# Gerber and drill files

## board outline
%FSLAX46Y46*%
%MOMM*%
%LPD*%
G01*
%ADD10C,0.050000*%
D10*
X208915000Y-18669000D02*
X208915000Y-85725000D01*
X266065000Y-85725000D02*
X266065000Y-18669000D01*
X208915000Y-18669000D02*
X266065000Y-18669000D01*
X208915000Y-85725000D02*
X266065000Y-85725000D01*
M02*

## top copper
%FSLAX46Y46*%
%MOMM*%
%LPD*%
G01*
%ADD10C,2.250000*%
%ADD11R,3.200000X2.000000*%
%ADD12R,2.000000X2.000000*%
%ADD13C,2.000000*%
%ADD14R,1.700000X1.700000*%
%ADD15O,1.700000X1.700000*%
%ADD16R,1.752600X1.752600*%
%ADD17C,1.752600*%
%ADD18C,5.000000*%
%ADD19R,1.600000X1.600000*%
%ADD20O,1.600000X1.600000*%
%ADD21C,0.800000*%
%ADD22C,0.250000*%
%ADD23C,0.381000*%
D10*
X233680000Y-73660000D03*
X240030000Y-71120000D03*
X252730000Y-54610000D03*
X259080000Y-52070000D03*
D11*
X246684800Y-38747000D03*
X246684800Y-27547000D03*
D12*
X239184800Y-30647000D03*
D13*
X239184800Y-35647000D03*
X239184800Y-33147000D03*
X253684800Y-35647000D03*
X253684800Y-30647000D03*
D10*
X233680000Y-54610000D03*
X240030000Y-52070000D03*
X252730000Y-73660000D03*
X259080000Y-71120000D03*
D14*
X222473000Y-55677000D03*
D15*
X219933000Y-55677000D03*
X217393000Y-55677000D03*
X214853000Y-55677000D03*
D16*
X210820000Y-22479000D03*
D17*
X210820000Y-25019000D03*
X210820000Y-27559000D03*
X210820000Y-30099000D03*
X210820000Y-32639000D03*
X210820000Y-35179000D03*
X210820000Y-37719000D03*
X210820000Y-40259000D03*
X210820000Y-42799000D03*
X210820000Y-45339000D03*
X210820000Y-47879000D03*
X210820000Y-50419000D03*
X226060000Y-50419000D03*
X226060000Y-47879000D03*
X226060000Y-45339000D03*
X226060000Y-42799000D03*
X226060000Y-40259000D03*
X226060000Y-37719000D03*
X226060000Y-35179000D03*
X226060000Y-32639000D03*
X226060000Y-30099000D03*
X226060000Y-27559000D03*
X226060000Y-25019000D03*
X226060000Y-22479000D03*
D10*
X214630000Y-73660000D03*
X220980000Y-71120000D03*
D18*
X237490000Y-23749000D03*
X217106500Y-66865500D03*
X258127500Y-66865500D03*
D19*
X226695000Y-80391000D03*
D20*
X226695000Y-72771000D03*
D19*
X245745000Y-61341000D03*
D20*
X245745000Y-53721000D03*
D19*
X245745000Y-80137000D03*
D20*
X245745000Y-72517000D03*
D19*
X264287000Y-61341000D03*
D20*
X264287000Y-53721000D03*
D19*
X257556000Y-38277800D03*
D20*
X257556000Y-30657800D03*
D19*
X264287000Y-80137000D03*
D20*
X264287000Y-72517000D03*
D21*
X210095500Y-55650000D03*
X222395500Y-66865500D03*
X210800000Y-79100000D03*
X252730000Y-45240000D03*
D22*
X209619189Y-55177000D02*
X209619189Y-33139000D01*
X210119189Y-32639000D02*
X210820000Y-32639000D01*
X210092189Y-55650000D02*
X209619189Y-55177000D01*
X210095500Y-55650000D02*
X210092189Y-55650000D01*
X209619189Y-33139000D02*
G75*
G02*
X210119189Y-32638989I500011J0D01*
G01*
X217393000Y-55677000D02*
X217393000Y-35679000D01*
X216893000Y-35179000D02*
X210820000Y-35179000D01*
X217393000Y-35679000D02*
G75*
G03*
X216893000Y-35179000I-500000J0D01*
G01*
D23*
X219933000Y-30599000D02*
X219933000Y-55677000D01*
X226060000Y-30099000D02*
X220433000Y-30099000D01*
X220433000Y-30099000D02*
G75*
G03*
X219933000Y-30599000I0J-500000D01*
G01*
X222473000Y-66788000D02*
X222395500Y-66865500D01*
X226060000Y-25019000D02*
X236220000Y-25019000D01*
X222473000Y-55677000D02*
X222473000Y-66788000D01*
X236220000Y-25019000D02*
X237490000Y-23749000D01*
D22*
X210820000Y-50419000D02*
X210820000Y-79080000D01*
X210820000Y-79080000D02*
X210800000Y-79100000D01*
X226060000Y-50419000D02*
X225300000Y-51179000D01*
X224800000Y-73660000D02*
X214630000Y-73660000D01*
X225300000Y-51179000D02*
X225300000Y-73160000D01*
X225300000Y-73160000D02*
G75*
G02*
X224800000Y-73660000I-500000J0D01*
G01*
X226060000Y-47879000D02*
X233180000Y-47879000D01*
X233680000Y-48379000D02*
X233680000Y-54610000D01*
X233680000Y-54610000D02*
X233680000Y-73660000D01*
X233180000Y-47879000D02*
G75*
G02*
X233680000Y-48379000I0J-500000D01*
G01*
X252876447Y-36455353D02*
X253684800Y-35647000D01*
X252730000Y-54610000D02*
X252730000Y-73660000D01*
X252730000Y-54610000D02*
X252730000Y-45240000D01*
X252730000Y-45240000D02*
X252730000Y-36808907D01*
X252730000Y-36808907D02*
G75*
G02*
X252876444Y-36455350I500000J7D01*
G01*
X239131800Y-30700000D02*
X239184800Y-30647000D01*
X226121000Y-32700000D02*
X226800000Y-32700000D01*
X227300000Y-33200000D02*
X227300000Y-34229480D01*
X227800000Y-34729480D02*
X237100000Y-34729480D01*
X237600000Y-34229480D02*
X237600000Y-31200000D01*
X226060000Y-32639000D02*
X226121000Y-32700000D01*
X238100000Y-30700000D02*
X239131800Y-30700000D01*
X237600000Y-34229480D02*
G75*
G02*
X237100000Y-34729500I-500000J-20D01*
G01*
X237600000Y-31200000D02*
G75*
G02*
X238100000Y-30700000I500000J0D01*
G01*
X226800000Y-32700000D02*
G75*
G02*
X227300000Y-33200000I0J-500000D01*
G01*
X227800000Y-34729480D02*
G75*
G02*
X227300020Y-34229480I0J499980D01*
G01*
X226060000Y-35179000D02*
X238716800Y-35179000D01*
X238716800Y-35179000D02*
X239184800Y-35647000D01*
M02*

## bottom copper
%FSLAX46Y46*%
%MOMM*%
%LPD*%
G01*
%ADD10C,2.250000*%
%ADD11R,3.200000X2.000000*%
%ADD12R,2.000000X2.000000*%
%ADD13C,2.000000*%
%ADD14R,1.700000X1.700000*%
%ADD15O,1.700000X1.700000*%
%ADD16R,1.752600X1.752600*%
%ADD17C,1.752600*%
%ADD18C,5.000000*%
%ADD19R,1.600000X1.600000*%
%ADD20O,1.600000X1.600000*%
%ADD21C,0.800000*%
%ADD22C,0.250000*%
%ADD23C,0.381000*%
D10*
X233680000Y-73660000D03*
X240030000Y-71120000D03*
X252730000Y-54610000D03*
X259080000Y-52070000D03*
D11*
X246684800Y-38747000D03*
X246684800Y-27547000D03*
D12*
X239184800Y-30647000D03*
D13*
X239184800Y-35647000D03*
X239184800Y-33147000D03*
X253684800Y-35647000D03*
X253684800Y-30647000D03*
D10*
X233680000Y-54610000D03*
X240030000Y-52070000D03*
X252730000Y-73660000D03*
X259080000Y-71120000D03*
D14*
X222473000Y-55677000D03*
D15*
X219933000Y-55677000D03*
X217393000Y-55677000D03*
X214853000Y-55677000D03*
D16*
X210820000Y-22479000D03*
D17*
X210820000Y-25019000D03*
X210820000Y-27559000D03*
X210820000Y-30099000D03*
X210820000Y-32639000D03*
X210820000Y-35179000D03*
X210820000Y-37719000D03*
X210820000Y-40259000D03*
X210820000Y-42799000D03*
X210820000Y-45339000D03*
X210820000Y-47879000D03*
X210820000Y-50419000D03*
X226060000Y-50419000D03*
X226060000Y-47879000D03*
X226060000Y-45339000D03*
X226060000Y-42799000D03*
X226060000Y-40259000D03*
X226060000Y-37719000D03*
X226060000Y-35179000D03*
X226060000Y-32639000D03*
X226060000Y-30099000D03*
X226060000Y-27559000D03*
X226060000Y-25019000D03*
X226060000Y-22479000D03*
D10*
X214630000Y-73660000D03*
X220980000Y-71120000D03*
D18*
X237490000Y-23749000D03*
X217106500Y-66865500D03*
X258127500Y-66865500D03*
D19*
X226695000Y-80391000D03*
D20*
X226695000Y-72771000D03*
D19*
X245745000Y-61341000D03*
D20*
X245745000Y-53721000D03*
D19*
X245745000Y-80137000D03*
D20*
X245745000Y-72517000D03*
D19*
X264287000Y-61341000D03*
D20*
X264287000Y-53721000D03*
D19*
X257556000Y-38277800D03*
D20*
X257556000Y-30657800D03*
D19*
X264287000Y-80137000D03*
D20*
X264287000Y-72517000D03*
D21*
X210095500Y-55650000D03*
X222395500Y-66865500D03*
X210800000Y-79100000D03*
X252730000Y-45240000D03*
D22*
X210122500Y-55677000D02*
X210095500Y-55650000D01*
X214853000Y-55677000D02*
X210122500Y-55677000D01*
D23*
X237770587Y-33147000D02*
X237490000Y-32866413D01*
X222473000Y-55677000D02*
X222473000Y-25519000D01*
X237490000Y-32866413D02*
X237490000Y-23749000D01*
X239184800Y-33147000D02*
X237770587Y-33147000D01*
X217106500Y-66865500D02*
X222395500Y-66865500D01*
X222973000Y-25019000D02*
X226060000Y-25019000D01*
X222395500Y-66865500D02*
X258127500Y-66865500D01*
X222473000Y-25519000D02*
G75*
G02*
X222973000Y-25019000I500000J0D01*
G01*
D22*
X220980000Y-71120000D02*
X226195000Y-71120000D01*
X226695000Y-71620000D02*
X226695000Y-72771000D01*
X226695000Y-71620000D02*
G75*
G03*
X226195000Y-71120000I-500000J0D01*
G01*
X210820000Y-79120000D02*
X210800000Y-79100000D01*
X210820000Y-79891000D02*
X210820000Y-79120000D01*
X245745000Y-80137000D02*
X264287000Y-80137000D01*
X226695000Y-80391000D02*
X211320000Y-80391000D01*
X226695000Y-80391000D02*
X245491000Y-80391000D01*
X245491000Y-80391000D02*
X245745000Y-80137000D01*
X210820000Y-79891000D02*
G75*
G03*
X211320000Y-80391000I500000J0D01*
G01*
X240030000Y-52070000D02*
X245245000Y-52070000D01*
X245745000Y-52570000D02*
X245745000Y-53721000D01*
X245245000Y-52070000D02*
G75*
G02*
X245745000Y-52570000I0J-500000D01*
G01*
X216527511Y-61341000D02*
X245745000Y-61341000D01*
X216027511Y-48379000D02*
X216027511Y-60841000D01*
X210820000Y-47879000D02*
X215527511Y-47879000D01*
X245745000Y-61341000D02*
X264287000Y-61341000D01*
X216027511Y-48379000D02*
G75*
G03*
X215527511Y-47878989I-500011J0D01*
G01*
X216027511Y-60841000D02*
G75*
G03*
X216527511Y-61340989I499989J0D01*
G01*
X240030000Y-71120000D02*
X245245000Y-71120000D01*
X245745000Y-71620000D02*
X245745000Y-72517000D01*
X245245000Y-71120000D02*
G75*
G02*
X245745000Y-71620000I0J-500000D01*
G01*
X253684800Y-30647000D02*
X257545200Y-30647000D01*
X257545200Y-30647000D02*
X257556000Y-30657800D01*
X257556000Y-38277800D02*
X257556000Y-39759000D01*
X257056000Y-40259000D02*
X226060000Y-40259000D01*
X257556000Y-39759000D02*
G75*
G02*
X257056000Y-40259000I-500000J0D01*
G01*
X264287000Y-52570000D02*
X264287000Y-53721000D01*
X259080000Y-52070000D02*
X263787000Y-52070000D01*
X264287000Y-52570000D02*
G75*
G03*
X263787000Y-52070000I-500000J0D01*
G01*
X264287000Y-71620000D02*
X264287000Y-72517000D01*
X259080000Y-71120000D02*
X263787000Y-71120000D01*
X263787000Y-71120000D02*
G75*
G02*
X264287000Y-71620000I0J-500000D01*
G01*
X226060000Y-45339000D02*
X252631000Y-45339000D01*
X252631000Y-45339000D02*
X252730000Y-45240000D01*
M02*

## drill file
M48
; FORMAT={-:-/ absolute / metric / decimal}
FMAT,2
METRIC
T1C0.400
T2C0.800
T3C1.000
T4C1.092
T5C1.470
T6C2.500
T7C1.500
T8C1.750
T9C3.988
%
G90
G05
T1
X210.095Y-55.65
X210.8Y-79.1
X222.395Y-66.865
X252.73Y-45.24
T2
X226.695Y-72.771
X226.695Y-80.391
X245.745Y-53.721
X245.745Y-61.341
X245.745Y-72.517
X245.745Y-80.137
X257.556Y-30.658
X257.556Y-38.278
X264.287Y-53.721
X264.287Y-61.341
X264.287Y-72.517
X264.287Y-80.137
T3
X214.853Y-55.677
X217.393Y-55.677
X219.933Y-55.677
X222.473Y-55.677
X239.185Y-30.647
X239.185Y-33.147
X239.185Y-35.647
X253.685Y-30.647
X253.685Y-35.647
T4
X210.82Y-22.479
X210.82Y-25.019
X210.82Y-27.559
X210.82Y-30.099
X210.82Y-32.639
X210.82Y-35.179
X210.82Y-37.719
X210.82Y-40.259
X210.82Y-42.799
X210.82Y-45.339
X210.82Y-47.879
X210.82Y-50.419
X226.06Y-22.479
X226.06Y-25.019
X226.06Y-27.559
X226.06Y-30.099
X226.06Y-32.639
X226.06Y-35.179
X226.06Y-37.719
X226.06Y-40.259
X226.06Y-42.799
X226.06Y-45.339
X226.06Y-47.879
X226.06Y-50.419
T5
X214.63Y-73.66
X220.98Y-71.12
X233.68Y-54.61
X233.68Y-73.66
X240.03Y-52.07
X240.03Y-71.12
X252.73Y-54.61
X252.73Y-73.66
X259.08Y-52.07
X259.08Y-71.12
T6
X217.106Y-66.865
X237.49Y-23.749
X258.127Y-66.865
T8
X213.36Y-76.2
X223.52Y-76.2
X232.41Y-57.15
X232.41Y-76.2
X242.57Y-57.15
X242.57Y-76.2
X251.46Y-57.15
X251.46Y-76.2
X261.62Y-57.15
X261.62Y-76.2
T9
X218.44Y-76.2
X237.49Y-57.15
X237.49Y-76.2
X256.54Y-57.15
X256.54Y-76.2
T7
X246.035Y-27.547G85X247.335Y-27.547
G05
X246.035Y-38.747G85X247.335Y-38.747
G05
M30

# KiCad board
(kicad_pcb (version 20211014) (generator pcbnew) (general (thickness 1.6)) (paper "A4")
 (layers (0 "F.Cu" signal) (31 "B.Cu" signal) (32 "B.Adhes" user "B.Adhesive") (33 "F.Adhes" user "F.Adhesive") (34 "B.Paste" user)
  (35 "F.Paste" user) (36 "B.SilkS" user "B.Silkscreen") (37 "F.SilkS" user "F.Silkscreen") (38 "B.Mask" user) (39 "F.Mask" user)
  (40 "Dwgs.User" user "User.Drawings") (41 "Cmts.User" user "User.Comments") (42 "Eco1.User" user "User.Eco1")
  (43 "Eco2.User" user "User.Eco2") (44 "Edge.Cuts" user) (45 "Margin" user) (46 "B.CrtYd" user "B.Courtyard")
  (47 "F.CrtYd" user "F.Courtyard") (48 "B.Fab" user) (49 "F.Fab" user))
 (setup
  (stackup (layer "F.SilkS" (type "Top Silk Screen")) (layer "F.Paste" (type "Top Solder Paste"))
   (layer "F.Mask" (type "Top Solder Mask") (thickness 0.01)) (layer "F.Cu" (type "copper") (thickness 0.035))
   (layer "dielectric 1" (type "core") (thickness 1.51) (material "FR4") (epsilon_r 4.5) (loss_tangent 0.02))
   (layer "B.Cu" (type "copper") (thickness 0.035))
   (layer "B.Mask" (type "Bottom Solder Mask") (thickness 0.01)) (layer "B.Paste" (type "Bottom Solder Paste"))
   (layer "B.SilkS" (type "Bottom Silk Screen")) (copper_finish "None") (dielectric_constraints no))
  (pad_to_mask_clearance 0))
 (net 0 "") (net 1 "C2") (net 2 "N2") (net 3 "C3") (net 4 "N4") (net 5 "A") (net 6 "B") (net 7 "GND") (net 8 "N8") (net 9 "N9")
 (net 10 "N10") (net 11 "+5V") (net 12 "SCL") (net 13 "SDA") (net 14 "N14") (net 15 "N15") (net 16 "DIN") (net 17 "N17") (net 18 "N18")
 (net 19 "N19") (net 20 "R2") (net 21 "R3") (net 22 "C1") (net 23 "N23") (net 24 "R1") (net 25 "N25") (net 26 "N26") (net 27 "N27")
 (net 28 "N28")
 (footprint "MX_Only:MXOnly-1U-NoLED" (layer "F.Cu") (at 237.49 76.2)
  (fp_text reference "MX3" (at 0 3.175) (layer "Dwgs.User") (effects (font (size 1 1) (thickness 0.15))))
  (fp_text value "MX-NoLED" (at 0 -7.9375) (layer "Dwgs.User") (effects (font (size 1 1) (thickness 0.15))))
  (pad "" np_thru_hole circle locked (at 5.08 0 48.0996) (size 1.75 1.75) (drill 1.75) (layers *.Cu *.Mask))
  (pad "" np_thru_hole circle locked (at 0 0) (size 3.9878 3.9878) (drill 3.9878) (layers *.Cu *.Mask))
  (pad "" np_thru_hole circle locked (at -5.08 0 48.0996) (size 1.75 1.75) (drill 1.75) (layers *.Cu *.Mask))
  (pad "1" thru_hole circle locked (at -3.81 -2.54) (size 2.25 2.25) (drill 1.47) (layers *.Cu "B.Mask") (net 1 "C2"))
  (pad "2" thru_hole circle locked (at 2.54 -5.08) (size 2.25 2.25) (drill 1.47) (layers *.Cu "B.Mask") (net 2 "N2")))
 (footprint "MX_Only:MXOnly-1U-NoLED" (layer "F.Cu") (at 256.54 57.15)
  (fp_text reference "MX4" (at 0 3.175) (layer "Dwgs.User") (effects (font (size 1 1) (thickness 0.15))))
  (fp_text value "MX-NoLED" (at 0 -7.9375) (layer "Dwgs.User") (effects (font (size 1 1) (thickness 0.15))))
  (pad "" np_thru_hole circle locked (at 5.08 0 48.0996) (size 1.75 1.75) (drill 1.75) (layers *.Cu *.Mask))
  (pad "" np_thru_hole circle locked (at 0 0) (size 3.9878 3.9878) (drill 3.9878) (layers *.Cu *.Mask))
  (pad "" np_thru_hole circle locked (at -5.08 0 48.0996) (size 1.75 1.75) (drill 1.75) (layers *.Cu *.Mask))
  (pad "1" thru_hole circle locked (at -3.81 -2.54) (size 2.25 2.25) (drill 1.47) (layers *.Cu "B.Mask") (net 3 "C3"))
  (pad "2" thru_hole circle locked (at 2.54 -5.08) (size 2.25 2.25) (drill 1.47) (layers *.Cu "B.Mask") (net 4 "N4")))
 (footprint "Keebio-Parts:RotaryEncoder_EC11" (layer "F.Cu") (at 246.6848 33.147)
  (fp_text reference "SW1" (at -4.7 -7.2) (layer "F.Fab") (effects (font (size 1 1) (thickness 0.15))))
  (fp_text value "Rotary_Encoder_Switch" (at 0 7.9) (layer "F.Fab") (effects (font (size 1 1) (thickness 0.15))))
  (pad "" np_thru_hole rect locked (at 0 5.6) (size 3.2 2) (drill oval 2.8 1.5) (layers *.Cu *.Mask))
  (pad "" np_thru_hole rect locked (at 0 -5.6) (size 3.2 2) (drill oval 2.8 1.5) (layers *.Cu *.Mask))
  (pad "A" thru_hole rect locked (at -7.5 -2.5) (size 2 2) (drill 1) (layers *.Cu *.Mask) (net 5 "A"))
  (pad "B" thru_hole circle locked (at -7.5 2.5) (size 2 2) (drill 1) (layers *.Cu *.Mask) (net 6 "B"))
  (pad "C" thru_hole circle locked (at -7.5 0) (size 2 2) (drill 1) (layers *.Cu *.Mask) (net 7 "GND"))
  (pad "S1" thru_hole circle locked (at 7 2.5) (size 2 2) (drill 1) (layers *.Cu *.Mask) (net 3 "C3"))
  (pad "S2" thru_hole circle locked (at 7 -2.5) (size 2 2) (drill 1) (layers *.Cu *.Mask) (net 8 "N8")))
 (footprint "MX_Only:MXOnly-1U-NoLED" (layer "F.Cu") (at 237.49 57.15)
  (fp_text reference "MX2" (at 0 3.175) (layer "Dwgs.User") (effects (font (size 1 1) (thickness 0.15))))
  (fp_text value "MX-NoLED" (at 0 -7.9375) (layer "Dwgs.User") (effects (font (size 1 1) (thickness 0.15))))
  (pad "" np_thru_hole circle locked (at -5.08 0 48.0996) (size 1.75 1.75) (drill 1.75) (layers *.Cu *.Mask))
  (pad "" np_thru_hole circle locked (at 5.08 0 48.0996) (size 1.75 1.75) (drill 1.75) (layers *.Cu *.Mask))
  (pad "" np_thru_hole circle locked (at 0 0) (size 3.9878 3.9878) (drill 3.9878) (layers *.Cu *.Mask))
  (pad "1" thru_hole circle locked (at -3.81 -2.54) (size 2.25 2.25) (drill 1.47) (layers *.Cu "B.Mask") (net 1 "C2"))
  (pad "2" thru_hole circle locked (at 2.54 -5.08) (size 2.25 2.25) (drill 1.47) (layers *.Cu "B.Mask") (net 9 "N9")))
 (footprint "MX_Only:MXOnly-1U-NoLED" (layer "F.Cu") (at 256.54 76.2)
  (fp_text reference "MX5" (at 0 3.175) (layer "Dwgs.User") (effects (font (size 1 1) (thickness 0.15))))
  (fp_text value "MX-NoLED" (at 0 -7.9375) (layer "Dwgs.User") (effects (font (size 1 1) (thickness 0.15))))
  (pad "" np_thru_hole circle locked (at 0 0) (size 3.9878 3.9878) (drill 3.9878) (layers *.Cu *.Mask))
  (pad "" np_thru_hole circle locked (at 5.08 0 48.0996) (size 1.75 1.75) (drill 1.75) (layers *.Cu *.Mask))
  (pad "" np_thru_hole circle locked (at -5.08 0 48.0996) (size 1.75 1.75) (drill 1.75) (layers *.Cu *.Mask))
  (pad "1" thru_hole circle locked (at -3.81 -2.54) (size 2.25 2.25) (drill 1.47) (layers *.Cu "B.Mask") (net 3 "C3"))
  (pad "2" thru_hole circle locked (at 2.54 -5.08) (size 2.25 2.25) (drill 1.47) (layers *.Cu "B.Mask") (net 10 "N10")))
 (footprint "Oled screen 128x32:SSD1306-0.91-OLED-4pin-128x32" (layer "F.Cu") (at 224.663 19.177 -90)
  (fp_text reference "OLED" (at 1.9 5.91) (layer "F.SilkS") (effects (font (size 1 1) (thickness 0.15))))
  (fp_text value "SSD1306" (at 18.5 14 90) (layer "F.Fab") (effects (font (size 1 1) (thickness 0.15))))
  (pad "1" thru_hole rect locked (at 36.5 2.19 270) (size 1.7 1.7) (drill 1) (layers *.Cu *.Mask) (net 7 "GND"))
  (pad "2" thru_hole oval locked (at 36.5 4.73 270) (size 1.7 1.7) (drill 1) (layers *.Cu *.Mask) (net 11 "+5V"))
  (pad "3" thru_hole oval locked (at 36.5 7.27 270) (size 1.7 1.7) (drill 1) (layers *.Cu *.Mask) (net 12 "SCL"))
  (pad "4" thru_hole oval locked (at 36.5 9.81 270) (size 1.7 1.7) (drill 1) (layers *.Cu *.Mask) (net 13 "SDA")))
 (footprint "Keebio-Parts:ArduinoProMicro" (layer "F.Cu") (at 218.44 36.449 -90)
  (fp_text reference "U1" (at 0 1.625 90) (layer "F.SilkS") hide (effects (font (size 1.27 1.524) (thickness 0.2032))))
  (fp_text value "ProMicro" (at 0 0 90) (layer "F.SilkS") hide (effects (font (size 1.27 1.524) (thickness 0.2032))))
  (pad "1" thru_hole rect locked (at -13.97 7.62 270) (size 1.7526 1.7526) (drill 1.0922) (layers *.Cu *.SilkS *.Mask) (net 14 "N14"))
  (pad "2" thru_hole circle locked (at -11.43 7.62 270) (size 1.7526 1.7526) (drill 1.0922) (layers *.Cu *.SilkS *.Mask) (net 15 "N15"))
  (pad "3" thru_hole circle locked (at -8.89 7.62 270) (size 1.7526 1.7526) (drill 1.0922) (layers *.Cu *.SilkS *.Mask) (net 7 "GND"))
  (pad "4" thru_hole circle locked (at -6.35 7.62 270) (size 1.7526 1.7526) (drill 1.0922) (layers *.Cu *.SilkS *.Mask) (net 7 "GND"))
  (pad "5" thru_hole circle locked (at -3.81 7.62 270) (size 1.7526 1.7526) (drill 1.0922) (layers *.Cu *.SilkS *.Mask) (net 13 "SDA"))
  (pad "6" thru_hole circle locked (at -1.27 7.62 270) (size 1.7526 1.7526) (drill 1.0922) (layers *.Cu *.SilkS *.Mask) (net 12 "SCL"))
  (pad "7" thru_hole circle locked (at 1.27 7.62 270) (size 1.7526 1.7526) (drill 1.0922) (layers *.Cu *.SilkS *.Mask) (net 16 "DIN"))
  (pad "8" thru_hole circle locked (at 3.81 7.62 270) (size 1.7526 1.7526) (drill 1.0922) (layers *.Cu *.SilkS *.Mask) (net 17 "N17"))
  (pad "9" thru_hole circle locked (at 6.35 7.62 270) (size 1.7526 1.7526) (drill 1.0922) (layers *.Cu *.SilkS *.Mask) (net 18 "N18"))
  (pad "10" thru_hole circle locked (at 8.89 7.62 270) (size 1.7526 1.7526) (drill 1.0922) (layers *.Cu *.SilkS *.Mask) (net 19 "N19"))
  (pad "11" thru_hole circle locked (at 11.43 7.62 270) (size 1.7526 1.7526) (drill 1.0922) (layers *.Cu *.SilkS *.Mask) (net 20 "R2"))
  (pad "12" thru_hole circle locked (at 13.97 7.62 270) (size 1.7526 1.7526) (drill 1.0922) (layers *.Cu *.SilkS *.Mask) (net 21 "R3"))
  (pad "13" thru_hole circle locked (at 13.97 -7.62 270) (size 1.7526 1.7526) (drill 1.0922) (layers *.Cu *.SilkS *.Mask) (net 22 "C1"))
  (pad "14" thru_hole circle locked (at 11.43 -7.62 270) (size 1.7526 1.7526) (drill 1.0922) (layers *.Cu *.SilkS *.Mask) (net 1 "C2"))
  (pad "15" thru_hole circle locked (at 8.89 -7.62 270) (size 1.7526 1.7526) (drill 1.0922) (layers *.Cu *.SilkS *.Mask) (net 3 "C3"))
  (pad "16" thru_hole circle locked (at 6.35 -7.62 270) (size 1.7526 1.7526) (drill 1.0922) (layers *.Cu *.SilkS *.Mask) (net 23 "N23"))
  (pad "17" thru_hole circle locked (at 3.81 -7.62 270) (size 1.7526 1.7526) (drill 1.0922) (layers *.Cu *.SilkS *.Mask) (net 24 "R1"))
  (pad "18" thru_hole circle locked (at 1.27 -7.62 270) (size 1.7526 1.7526) (drill 1.0922) (layers *.Cu *.SilkS *.Mask) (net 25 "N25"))
  (pad "19" thru_hole circle locked (at -1.27 -7.62 270) (size 1.7526 1.7526) (drill 1.0922) (layers *.Cu *.SilkS *.Mask) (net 6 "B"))
  (pad "20" thru_hole circle locked (at -3.81 -7.62 270) (size 1.7526 1.7526) (drill 1.0922) (layers *.Cu *.SilkS *.Mask) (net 5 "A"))
  (pad "21" thru_hole circle locked (at -6.35 -7.62 270) (size 1.7526 1.7526) (drill 1.0922) (layers *.Cu *.SilkS *.Mask) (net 11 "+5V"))
  (pad "22" thru_hole circle locked (at -8.89 -7.62 270) (size 1.7526 1.7526) (drill 1.0922) (layers *.Cu *.SilkS *.Mask) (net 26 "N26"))
  (pad "23" thru_hole circle locked (at -11.43 -7.62 270) (size 1.7526 1.7526) (drill 1.0922) (layers *.Cu *.SilkS *.Mask) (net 7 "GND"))
  (pad "24" thru_hole circle locked (at -13.97 -7.62 270) (size 1.7526 1.7526) (drill 1.0922) (layers *.Cu *.SilkS *.Mask) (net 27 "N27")))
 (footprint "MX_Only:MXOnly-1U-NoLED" (layer "F.Cu") (at 218.44 76.2)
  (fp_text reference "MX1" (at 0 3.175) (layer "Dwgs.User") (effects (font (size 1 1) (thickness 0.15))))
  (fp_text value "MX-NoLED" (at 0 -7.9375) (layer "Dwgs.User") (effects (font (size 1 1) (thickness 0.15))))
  (pad "" np_thru_hole circle locked (at 5.08 0 48.0996) (size 1.75 1.75) (drill 1.75) (layers *.Cu *.Mask))
  (pad "" np_thru_hole circle locked (at -5.08 0 48.0996) (size 1.75 1.75) (drill 1.75) (layers *.Cu *.Mask))
  (pad "" np_thru_hole circle locked (at 0 0) (size 3.9878 3.9878) (drill 3.9878) (layers *.Cu *.Mask))
  (pad "1" thru_hole circle locked (at -3.81 -2.54) (size 2.25 2.25) (drill 1.47) (layers *.Cu "B.Mask") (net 22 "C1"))
  (pad "2" thru_hole circle locked (at 2.54 -5.08) (size 2.25 2.25) (drill 1.47) (layers *.Cu "B.Mask") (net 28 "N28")))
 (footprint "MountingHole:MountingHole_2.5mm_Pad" (layer "F.Cu") (at 237.49 23.749)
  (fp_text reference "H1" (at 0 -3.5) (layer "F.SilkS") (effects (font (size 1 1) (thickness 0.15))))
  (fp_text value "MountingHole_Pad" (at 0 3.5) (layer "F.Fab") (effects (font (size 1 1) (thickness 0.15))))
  (pad "1" thru_hole circle locked (at 0 0) (size 5 5) (drill 2.5) (layers *.Cu *.Mask) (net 7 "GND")))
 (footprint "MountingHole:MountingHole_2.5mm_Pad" (layer "F.Cu") (at 217.1065 66.8655)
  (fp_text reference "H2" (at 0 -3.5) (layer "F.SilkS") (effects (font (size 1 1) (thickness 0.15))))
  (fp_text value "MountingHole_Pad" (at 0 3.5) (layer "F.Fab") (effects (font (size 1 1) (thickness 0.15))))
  (pad "1" thru_hole circle locked (at 0 0) (size 5 5) (drill 2.5) (layers *.Cu *.Mask) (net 7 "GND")))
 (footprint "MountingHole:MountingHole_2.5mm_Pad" (layer "F.Cu") (at 258.1275 66.8655)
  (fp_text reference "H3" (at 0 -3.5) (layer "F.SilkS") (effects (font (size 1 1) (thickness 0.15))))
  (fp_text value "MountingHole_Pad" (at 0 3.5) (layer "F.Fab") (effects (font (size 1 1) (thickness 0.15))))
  (pad "1" thru_hole circle locked (at 0 0) (size 5 5) (drill 2.5) (layers *.Cu *.Mask) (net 7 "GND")))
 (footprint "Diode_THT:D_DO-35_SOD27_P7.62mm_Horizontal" (layer "B.Cu") (at 226.695 80.391 90)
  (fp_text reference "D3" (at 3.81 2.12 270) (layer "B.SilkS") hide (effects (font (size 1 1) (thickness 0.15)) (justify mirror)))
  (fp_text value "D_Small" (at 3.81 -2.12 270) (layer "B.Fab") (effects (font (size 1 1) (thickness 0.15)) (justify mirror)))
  (pad "1" thru_hole rect locked (at 0 0 90) (size 1.6 1.6) (drill 0.8) (layers *.Cu *.Mask) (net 21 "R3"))
  (pad "2" thru_hole oval locked (at 7.62 0 90) (size 1.6 1.6) (drill 0.8) (layers *.Cu *.Mask) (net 28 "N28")))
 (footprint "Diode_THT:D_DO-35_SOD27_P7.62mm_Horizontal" (layer "B.Cu") (at 245.745 61.341 90)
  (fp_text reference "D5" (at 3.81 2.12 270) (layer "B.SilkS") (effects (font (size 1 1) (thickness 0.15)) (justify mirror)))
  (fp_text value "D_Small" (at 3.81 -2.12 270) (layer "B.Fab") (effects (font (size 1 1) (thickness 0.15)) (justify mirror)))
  (pad "1" thru_hole rect locked (at 0 0 90) (size 1.6 1.6) (drill 0.8) (layers *.Cu *.Mask) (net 20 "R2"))
  (pad "2" thru_hole oval locked (at 7.62 0 90) (size 1.6 1.6) (drill 0.8) (layers *.Cu *.Mask) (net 9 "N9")))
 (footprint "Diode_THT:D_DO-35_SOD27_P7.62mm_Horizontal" (layer "B.Cu") (at 245.745 80.137 90)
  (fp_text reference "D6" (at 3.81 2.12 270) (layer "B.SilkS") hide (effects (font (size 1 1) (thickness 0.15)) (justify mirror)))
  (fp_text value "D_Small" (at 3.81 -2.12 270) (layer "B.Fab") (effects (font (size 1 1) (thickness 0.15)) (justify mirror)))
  (pad "1" thru_hole rect locked (at 0 0 90) (size 1.6 1.6) (drill 0.8) (layers *.Cu *.Mask) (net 21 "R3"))
  (pad "2" thru_hole oval locked (at 7.62 0 90) (size 1.6 1.6) (drill 0.8) (layers *.Cu *.Mask) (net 2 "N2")))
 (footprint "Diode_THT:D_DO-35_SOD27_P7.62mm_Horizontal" (layer "B.Cu") (at 264.287 61.341 90)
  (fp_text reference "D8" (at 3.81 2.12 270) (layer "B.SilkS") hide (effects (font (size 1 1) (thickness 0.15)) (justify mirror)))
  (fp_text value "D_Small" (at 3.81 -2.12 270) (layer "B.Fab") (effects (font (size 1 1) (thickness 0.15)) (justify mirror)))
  (pad "1" thru_hole rect locked (at 0 0 90) (size 1.6 1.6) (drill 0.8) (layers *.Cu *.Mask) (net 20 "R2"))
  (pad "2" thru_hole oval locked (at 7.62 0 90) (size 1.6 1.6) (drill 0.8) (layers *.Cu *.Mask) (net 4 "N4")))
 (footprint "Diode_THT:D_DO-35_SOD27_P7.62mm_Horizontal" (layer "B.Cu") (at 257.556 38.2778 90)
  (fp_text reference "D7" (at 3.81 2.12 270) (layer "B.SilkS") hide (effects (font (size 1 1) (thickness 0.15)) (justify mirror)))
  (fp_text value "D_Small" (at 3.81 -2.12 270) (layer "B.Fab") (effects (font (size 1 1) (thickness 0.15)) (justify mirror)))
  (pad "1" thru_hole rect locked (at 0 0 90) (size 1.6 1.6) (drill 0.8) (layers *.Cu *.Mask) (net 24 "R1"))
  (pad "2" thru_hole oval locked (at 7.62 0 90) (size 1.6 1.6) (drill 0.8) (layers *.Cu *.Mask) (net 8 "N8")))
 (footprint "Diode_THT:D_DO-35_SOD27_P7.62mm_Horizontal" (layer "B.Cu") (at 264.287 80.137 90)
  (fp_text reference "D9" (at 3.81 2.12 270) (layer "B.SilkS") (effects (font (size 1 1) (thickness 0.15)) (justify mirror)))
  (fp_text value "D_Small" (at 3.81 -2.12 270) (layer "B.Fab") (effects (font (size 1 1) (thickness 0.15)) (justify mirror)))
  (pad "1" thru_hole rect locked (at 0 0 90) (size 1.6 1.6) (drill 0.8) (layers *.Cu *.Mask) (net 21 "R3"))
  (pad "2" thru_hole oval locked (at 7.62 0 90) (size 1.6 1.6) (drill 0.8) (layers *.Cu *.Mask) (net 10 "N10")))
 (gr_line (start 208.915 18.669) (end 208.915 85.725) (layer "Edge.Cuts") (width 0.05))
 (gr_line (start 266.065 85.725) (end 266.065 18.669) (layer "Edge.Cuts") (width 0.05))
 (gr_line (start 208.915 18.669) (end 266.065 18.669) (layer "Edge.Cuts") (width 0.05))
 (gr_line (start 208.915 85.725) (end 266.065 85.725) (layer "Edge.Cuts") (width 0.05))
 (segment (start 209.619189 55.177) (end 209.619189 33.139) (width 0.25) (layer "F.Cu") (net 13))
 (segment (start 210.119189 32.639) (end 210.82 32.639) (width 0.25) (layer "F.Cu") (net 13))
 (segment (start 210.092189 55.65) (end 209.619189 55.177) (width 0.25) (layer "F.Cu") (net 13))
 (segment (start 210.0955 55.65) (end 210.092189 55.65) (width 0.25) (layer "F.Cu") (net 13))
 (via (at 210.0955 55.65) (size 0.8) (drill 0.4) (layers "F.Cu" "B.Cu") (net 13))
 (arc (start 209.619189 33.139) (mid 209.765636 32.785447) (end 210.119189 32.639) (width 0.25) (layer "F.Cu") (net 13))
 (segment (start 210.1225 55.677) (end 210.0955 55.65) (width 0.25) (layer "B.Cu") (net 13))
 (segment (start 214.853 55.677) (end 210.1225 55.677) (width 0.25) (layer "B.Cu") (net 13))
 (segment (start 217.393 55.677) (end 217.393 35.679) (width 0.25) (layer "F.Cu") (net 12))
 (segment (start 216.893 35.179) (end 210.82 35.179) (width 0.25) (layer "F.Cu") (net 12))
 (arc (start 217.393 35.679) (mid 217.246553 35.325447) (end 216.893 35.179) (width 0.25) (layer "F.Cu") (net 12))
 (segment (start 219.933 30.599) (end 219.933 55.677) (width 0.381) (layer "F.Cu") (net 11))
 (segment (start 226.06 30.099) (end 220.433 30.099) (width 0.381) (layer "F.Cu") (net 11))
 (arc (start 220.433 30.099) (mid 220.079447 30.245447) (end 219.933 30.599) (width 0.381) (layer "F.Cu") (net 11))
 (segment (start 222.473 66.788) (end 222.3955 66.8655) (width 0.381) (layer "F.Cu") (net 7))
 (segment (start 226.06 25.019) (end 236.22 25.019) (width 0.381) (layer "F.Cu") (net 7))
 (segment (start 222.473 55.677) (end 222.473 66.788) (width 0.381) (layer "F.Cu") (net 7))
 (segment (start 236.22 25.019) (end 237.49 23.749) (width 0.381) (layer "F.Cu") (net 7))
 (via (at 222.3955 66.8655) (size 0.8) (drill 0.4) (layers "F.Cu" "B.Cu") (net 7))
 (segment (start 237.770587 33.147) (end 237.49 32.866413) (width 0.381) (layer "B.Cu") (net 7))
 (segment (start 222.473 55.677) (end 222.473 25.519) (width 0.381) (layer "B.Cu") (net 7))
 (segment (start 237.49 32.866413) (end 237.49 23.749) (width 0.381) (layer "B.Cu") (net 7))
 (segment (start 239.1848 33.147) (end 237.770587 33.147) (width 0.381) (layer "B.Cu") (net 7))
 (segment (start 217.1065 66.8655) (end 222.3955 66.8655) (width 0.381) (layer "B.Cu") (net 7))
 (segment (start 222.973 25.019) (end 226.06 25.019) (width 0.381) (layer "B.Cu") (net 7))
 (segment (start 222.3955 66.8655) (end 258.1275 66.8655) (width 0.381) (layer "B.Cu") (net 7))
 (arc (start 222.473 25.519) (mid 222.619447 25.165447) (end 222.973 25.019) (width 0.381) (layer "B.Cu") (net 7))
 (segment (start 220.98 71.12) (end 226.195 71.12) (width 0.25) (layer "B.Cu") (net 28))
 (segment (start 226.695 71.62) (end 226.695 72.771) (width 0.25) (layer "B.Cu") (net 28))
 (arc (start 226.695 71.62) (mid 226.548553 71.266447) (end 226.195 71.12) (width 0.25) (layer "B.Cu") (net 28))
 (segment (start 210.82 50.419) (end 210.82 79.08) (width 0.25) (layer "F.Cu") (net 21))
 (segment (start 210.82 79.08) (end 210.8 79.1) (width 0.25) (layer "F.Cu") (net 21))
 (via (at 210.8 79.1) (size 0.8) (drill 0.4) (layers "F.Cu" "B.Cu") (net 21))
 (segment (start 210.82 79.12) (end 210.8 79.1) (width 0.25) (layer "B.Cu") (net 21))
 (segment (start 210.82 79.891) (end 210.82 79.12) (width 0.25) (layer "B.Cu") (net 21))
 (segment (start 245.745 80.137) (end 264.287 80.137) (width 0.25) (layer "B.Cu") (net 21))
 (segment (start 226.695 80.391) (end 211.32 80.391) (width 0.25) (layer "B.Cu") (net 21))
 (segment (start 226.695 80.391) (end 245.491 80.391) (width 0.25) (layer "B.Cu") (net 21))
 (segment (start 245.491 80.391) (end 245.745 80.137) (width 0.25) (layer "B.Cu") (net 21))
 (arc (start 210.82 79.891) (mid 210.966447 80.244553) (end 211.32 80.391) (width 0.25) (layer "B.Cu") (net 21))
 (segment (start 240.03 52.07) (end 245.245 52.07) (width 0.25) (layer "B.Cu") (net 9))
 (segment (start 245.745 52.57) (end 245.745 53.721) (width 0.25) (layer "B.Cu") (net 9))
 (arc (start 245.245 52.07) (mid 245.598553 52.216447) (end 245.745 52.57) (width 0.25) (layer "B.Cu") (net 9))
 (segment (start 216.527511 61.341) (end 245.745 61.341) (width 0.25) (layer "B.Cu") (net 20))
 (segment (start 216.027511 48.379) (end 216.027511 60.841) (width 0.25) (layer "B.Cu") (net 20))
 (segment (start 210.82 47.879) (end 215.527511 47.879) (width 0.25) (layer "B.Cu") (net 20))
 (segment (start 245.745 61.341) (end 264.287 61.341) (width 0.25) (layer "B.Cu") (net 20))
 (arc (start 216.027511 48.379) (mid 215.881064 48.025447) (end 215.527511 47.879) (width 0.25) (layer "B.Cu") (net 20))
 (arc (start 216.027511 60.841) (mid 216.173958 61.194553) (end 216.527511 61.341) (width 0.25) (layer "B.Cu") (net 20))
 (segment (start 240.03 71.12) (end 245.245 71.12) (width 0.25) (layer "B.Cu") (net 2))
 (segment (start 245.745 71.62) (end 245.745 72.517) (width 0.25) (layer "B.Cu") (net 2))
 (arc (start 245.245 71.12) (mid 245.598553 71.266447) (end 245.745 71.62) (width 0.25) (layer "B.Cu") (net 2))
 (segment (start 253.6848 30.647) (end 257.5452 30.647) (width 0.25) (layer "B.Cu") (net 8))
 (segment (start 257.5452 30.647) (end 257.556 30.6578) (width 0.25) (layer "B.Cu") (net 8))
 (segment (start 257.556 38.2778) (end 257.556 39.759) (width 0.25) (layer "B.Cu") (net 24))
 (segment (start 257.056 40.259) (end 226.06 40.259) (width 0.25) (layer "B.Cu") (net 24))
 (arc (start 257.556 39.759) (mid 257.409553 40.112553) (end 257.056 40.259) (width 0.25) (layer "B.Cu") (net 24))
 (segment (start 264.287 52.57) (end 264.287 53.721) (width 0.25) (layer "B.Cu") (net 4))
 (segment (start 259.08 52.07) (end 263.787 52.07) (width 0.25) (layer "B.Cu") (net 4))
 (arc (start 264.287 52.57) (mid 264.140553 52.216447) (end 263.787 52.07) (width 0.25) (layer "B.Cu") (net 4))
 (segment (start 264.287 71.62) (end 264.287 72.517) (width 0.25) (layer "B.Cu") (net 10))
 (segment (start 259.08 71.12) (end 263.787 71.12) (width 0.25) (layer "B.Cu") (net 10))
 (arc (start 263.787 71.12) (mid 264.140553 71.266447) (end 264.287 71.62) (width 0.25) (layer "B.Cu") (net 10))
 (segment (start 226.06 50.419) (end 225.3 51.179) (width 0.25) (layer "F.Cu") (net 22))
 (segment (start 224.8 73.66) (end 214.63 73.66) (width 0.25) (layer "F.Cu") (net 22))
 (segment (start 225.3 51.179) (end 225.3 73.16) (width 0.25) (layer "F.Cu") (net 22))
 (arc (start 225.3 73.16) (mid 225.153553 73.513553) (end 224.8 73.66) (width 0.25) (layer "F.Cu") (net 22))
 (segment (start 226.06 47.879) (end 233.18 47.879) (width 0.25) (layer "F.Cu") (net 1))
 (segment (start 233.68 48.379) (end 233.68 54.61) (width 0.25) (layer "F.Cu") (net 1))
 (segment (start 233.68 54.61) (end 233.68 73.66) (width 0.25) (layer "F.Cu") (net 1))
 (arc (start 233.18 47.879) (mid 233.533553 48.025447) (end 233.68 48.379) (width 0.25) (layer "F.Cu") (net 1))
 (segment (start 252.876447 36.455353) (end 253.6848 35.647) (width 0.25) (layer "F.Cu") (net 3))
 (segment (start 252.73 54.61) (end 252.73 73.66) (width 0.25) (layer "F.Cu") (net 3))
 (segment (start 252.73 54.61) (end 252.73 45.24) (width 0.25) (layer "F.Cu") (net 3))
 (segment (start 252.73 45.24) (end 252.73 36.808907) (width 0.25) (layer "F.Cu") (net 3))
 (via (at 252.73 45.24) (size 0.8) (drill 0.4) (layers "F.Cu" "B.Cu") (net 3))
 (arc (start 252.73 36.808907) (mid 252.76806 36.617565) (end 252.876447 36.455353) (width 0.25) (layer "F.Cu") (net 3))
 (segment (start 226.06 45.339) (end 252.631 45.339) (width 0.25) (layer "B.Cu") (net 3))
 (segment (start 252.631 45.339) (end 252.73 45.24) (width 0.25) (layer "B.Cu") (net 3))
 (segment (start 239.1318 30.7) (end 239.1848 30.647) (width 0.25) (layer "F.Cu") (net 5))
 (segment (start 226.121 32.7) (end 226.8 32.7) (width 0.25) (layer "F.Cu") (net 5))
 (segment (start 227.3 33.2) (end 227.3 34.22948) (width 0.25) (layer "F.Cu") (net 5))
 (segment (start 227.8 34.72948) (end 237.1 34.72948) (width 0.25) (layer "F.Cu") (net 5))
 (segment (start 237.6 34.22948) (end 237.6 31.2) (width 0.25) (layer "F.Cu") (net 5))
 (segment (start 226.06 32.639) (end 226.121 32.7) (width 0.25) (layer "F.Cu") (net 5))
 (segment (start 238.1 30.7) (end 239.1318 30.7) (width 0.25) (layer "F.Cu") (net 5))
 (arc (start 237.6 34.22948) (mid 237.453553 34.583033) (end 237.1 34.72948) (width 0.25) (layer "F.Cu") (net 5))
 (arc (start 237.6 31.2) (mid 237.746447 30.846447) (end 238.1 30.7) (width 0.25) (layer "F.Cu") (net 5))
 (arc (start 226.8 32.7) (mid 227.153553 32.846447) (end 227.3 33.2) (width 0.25) (layer "F.Cu") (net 5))
 (arc (start 227.8 34.72948) (mid 227.446447 34.583033) (end 227.3 34.22948) (width 0.25) (layer "F.Cu") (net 5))
 (segment (start 226.06 35.179) (end 238.7168 35.179) (width 0.25) (layer "F.Cu") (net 6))
 (segment (start 238.7168 35.179) (end 239.1848 35.647) (width 0.25) (layer "F.Cu") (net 6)))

